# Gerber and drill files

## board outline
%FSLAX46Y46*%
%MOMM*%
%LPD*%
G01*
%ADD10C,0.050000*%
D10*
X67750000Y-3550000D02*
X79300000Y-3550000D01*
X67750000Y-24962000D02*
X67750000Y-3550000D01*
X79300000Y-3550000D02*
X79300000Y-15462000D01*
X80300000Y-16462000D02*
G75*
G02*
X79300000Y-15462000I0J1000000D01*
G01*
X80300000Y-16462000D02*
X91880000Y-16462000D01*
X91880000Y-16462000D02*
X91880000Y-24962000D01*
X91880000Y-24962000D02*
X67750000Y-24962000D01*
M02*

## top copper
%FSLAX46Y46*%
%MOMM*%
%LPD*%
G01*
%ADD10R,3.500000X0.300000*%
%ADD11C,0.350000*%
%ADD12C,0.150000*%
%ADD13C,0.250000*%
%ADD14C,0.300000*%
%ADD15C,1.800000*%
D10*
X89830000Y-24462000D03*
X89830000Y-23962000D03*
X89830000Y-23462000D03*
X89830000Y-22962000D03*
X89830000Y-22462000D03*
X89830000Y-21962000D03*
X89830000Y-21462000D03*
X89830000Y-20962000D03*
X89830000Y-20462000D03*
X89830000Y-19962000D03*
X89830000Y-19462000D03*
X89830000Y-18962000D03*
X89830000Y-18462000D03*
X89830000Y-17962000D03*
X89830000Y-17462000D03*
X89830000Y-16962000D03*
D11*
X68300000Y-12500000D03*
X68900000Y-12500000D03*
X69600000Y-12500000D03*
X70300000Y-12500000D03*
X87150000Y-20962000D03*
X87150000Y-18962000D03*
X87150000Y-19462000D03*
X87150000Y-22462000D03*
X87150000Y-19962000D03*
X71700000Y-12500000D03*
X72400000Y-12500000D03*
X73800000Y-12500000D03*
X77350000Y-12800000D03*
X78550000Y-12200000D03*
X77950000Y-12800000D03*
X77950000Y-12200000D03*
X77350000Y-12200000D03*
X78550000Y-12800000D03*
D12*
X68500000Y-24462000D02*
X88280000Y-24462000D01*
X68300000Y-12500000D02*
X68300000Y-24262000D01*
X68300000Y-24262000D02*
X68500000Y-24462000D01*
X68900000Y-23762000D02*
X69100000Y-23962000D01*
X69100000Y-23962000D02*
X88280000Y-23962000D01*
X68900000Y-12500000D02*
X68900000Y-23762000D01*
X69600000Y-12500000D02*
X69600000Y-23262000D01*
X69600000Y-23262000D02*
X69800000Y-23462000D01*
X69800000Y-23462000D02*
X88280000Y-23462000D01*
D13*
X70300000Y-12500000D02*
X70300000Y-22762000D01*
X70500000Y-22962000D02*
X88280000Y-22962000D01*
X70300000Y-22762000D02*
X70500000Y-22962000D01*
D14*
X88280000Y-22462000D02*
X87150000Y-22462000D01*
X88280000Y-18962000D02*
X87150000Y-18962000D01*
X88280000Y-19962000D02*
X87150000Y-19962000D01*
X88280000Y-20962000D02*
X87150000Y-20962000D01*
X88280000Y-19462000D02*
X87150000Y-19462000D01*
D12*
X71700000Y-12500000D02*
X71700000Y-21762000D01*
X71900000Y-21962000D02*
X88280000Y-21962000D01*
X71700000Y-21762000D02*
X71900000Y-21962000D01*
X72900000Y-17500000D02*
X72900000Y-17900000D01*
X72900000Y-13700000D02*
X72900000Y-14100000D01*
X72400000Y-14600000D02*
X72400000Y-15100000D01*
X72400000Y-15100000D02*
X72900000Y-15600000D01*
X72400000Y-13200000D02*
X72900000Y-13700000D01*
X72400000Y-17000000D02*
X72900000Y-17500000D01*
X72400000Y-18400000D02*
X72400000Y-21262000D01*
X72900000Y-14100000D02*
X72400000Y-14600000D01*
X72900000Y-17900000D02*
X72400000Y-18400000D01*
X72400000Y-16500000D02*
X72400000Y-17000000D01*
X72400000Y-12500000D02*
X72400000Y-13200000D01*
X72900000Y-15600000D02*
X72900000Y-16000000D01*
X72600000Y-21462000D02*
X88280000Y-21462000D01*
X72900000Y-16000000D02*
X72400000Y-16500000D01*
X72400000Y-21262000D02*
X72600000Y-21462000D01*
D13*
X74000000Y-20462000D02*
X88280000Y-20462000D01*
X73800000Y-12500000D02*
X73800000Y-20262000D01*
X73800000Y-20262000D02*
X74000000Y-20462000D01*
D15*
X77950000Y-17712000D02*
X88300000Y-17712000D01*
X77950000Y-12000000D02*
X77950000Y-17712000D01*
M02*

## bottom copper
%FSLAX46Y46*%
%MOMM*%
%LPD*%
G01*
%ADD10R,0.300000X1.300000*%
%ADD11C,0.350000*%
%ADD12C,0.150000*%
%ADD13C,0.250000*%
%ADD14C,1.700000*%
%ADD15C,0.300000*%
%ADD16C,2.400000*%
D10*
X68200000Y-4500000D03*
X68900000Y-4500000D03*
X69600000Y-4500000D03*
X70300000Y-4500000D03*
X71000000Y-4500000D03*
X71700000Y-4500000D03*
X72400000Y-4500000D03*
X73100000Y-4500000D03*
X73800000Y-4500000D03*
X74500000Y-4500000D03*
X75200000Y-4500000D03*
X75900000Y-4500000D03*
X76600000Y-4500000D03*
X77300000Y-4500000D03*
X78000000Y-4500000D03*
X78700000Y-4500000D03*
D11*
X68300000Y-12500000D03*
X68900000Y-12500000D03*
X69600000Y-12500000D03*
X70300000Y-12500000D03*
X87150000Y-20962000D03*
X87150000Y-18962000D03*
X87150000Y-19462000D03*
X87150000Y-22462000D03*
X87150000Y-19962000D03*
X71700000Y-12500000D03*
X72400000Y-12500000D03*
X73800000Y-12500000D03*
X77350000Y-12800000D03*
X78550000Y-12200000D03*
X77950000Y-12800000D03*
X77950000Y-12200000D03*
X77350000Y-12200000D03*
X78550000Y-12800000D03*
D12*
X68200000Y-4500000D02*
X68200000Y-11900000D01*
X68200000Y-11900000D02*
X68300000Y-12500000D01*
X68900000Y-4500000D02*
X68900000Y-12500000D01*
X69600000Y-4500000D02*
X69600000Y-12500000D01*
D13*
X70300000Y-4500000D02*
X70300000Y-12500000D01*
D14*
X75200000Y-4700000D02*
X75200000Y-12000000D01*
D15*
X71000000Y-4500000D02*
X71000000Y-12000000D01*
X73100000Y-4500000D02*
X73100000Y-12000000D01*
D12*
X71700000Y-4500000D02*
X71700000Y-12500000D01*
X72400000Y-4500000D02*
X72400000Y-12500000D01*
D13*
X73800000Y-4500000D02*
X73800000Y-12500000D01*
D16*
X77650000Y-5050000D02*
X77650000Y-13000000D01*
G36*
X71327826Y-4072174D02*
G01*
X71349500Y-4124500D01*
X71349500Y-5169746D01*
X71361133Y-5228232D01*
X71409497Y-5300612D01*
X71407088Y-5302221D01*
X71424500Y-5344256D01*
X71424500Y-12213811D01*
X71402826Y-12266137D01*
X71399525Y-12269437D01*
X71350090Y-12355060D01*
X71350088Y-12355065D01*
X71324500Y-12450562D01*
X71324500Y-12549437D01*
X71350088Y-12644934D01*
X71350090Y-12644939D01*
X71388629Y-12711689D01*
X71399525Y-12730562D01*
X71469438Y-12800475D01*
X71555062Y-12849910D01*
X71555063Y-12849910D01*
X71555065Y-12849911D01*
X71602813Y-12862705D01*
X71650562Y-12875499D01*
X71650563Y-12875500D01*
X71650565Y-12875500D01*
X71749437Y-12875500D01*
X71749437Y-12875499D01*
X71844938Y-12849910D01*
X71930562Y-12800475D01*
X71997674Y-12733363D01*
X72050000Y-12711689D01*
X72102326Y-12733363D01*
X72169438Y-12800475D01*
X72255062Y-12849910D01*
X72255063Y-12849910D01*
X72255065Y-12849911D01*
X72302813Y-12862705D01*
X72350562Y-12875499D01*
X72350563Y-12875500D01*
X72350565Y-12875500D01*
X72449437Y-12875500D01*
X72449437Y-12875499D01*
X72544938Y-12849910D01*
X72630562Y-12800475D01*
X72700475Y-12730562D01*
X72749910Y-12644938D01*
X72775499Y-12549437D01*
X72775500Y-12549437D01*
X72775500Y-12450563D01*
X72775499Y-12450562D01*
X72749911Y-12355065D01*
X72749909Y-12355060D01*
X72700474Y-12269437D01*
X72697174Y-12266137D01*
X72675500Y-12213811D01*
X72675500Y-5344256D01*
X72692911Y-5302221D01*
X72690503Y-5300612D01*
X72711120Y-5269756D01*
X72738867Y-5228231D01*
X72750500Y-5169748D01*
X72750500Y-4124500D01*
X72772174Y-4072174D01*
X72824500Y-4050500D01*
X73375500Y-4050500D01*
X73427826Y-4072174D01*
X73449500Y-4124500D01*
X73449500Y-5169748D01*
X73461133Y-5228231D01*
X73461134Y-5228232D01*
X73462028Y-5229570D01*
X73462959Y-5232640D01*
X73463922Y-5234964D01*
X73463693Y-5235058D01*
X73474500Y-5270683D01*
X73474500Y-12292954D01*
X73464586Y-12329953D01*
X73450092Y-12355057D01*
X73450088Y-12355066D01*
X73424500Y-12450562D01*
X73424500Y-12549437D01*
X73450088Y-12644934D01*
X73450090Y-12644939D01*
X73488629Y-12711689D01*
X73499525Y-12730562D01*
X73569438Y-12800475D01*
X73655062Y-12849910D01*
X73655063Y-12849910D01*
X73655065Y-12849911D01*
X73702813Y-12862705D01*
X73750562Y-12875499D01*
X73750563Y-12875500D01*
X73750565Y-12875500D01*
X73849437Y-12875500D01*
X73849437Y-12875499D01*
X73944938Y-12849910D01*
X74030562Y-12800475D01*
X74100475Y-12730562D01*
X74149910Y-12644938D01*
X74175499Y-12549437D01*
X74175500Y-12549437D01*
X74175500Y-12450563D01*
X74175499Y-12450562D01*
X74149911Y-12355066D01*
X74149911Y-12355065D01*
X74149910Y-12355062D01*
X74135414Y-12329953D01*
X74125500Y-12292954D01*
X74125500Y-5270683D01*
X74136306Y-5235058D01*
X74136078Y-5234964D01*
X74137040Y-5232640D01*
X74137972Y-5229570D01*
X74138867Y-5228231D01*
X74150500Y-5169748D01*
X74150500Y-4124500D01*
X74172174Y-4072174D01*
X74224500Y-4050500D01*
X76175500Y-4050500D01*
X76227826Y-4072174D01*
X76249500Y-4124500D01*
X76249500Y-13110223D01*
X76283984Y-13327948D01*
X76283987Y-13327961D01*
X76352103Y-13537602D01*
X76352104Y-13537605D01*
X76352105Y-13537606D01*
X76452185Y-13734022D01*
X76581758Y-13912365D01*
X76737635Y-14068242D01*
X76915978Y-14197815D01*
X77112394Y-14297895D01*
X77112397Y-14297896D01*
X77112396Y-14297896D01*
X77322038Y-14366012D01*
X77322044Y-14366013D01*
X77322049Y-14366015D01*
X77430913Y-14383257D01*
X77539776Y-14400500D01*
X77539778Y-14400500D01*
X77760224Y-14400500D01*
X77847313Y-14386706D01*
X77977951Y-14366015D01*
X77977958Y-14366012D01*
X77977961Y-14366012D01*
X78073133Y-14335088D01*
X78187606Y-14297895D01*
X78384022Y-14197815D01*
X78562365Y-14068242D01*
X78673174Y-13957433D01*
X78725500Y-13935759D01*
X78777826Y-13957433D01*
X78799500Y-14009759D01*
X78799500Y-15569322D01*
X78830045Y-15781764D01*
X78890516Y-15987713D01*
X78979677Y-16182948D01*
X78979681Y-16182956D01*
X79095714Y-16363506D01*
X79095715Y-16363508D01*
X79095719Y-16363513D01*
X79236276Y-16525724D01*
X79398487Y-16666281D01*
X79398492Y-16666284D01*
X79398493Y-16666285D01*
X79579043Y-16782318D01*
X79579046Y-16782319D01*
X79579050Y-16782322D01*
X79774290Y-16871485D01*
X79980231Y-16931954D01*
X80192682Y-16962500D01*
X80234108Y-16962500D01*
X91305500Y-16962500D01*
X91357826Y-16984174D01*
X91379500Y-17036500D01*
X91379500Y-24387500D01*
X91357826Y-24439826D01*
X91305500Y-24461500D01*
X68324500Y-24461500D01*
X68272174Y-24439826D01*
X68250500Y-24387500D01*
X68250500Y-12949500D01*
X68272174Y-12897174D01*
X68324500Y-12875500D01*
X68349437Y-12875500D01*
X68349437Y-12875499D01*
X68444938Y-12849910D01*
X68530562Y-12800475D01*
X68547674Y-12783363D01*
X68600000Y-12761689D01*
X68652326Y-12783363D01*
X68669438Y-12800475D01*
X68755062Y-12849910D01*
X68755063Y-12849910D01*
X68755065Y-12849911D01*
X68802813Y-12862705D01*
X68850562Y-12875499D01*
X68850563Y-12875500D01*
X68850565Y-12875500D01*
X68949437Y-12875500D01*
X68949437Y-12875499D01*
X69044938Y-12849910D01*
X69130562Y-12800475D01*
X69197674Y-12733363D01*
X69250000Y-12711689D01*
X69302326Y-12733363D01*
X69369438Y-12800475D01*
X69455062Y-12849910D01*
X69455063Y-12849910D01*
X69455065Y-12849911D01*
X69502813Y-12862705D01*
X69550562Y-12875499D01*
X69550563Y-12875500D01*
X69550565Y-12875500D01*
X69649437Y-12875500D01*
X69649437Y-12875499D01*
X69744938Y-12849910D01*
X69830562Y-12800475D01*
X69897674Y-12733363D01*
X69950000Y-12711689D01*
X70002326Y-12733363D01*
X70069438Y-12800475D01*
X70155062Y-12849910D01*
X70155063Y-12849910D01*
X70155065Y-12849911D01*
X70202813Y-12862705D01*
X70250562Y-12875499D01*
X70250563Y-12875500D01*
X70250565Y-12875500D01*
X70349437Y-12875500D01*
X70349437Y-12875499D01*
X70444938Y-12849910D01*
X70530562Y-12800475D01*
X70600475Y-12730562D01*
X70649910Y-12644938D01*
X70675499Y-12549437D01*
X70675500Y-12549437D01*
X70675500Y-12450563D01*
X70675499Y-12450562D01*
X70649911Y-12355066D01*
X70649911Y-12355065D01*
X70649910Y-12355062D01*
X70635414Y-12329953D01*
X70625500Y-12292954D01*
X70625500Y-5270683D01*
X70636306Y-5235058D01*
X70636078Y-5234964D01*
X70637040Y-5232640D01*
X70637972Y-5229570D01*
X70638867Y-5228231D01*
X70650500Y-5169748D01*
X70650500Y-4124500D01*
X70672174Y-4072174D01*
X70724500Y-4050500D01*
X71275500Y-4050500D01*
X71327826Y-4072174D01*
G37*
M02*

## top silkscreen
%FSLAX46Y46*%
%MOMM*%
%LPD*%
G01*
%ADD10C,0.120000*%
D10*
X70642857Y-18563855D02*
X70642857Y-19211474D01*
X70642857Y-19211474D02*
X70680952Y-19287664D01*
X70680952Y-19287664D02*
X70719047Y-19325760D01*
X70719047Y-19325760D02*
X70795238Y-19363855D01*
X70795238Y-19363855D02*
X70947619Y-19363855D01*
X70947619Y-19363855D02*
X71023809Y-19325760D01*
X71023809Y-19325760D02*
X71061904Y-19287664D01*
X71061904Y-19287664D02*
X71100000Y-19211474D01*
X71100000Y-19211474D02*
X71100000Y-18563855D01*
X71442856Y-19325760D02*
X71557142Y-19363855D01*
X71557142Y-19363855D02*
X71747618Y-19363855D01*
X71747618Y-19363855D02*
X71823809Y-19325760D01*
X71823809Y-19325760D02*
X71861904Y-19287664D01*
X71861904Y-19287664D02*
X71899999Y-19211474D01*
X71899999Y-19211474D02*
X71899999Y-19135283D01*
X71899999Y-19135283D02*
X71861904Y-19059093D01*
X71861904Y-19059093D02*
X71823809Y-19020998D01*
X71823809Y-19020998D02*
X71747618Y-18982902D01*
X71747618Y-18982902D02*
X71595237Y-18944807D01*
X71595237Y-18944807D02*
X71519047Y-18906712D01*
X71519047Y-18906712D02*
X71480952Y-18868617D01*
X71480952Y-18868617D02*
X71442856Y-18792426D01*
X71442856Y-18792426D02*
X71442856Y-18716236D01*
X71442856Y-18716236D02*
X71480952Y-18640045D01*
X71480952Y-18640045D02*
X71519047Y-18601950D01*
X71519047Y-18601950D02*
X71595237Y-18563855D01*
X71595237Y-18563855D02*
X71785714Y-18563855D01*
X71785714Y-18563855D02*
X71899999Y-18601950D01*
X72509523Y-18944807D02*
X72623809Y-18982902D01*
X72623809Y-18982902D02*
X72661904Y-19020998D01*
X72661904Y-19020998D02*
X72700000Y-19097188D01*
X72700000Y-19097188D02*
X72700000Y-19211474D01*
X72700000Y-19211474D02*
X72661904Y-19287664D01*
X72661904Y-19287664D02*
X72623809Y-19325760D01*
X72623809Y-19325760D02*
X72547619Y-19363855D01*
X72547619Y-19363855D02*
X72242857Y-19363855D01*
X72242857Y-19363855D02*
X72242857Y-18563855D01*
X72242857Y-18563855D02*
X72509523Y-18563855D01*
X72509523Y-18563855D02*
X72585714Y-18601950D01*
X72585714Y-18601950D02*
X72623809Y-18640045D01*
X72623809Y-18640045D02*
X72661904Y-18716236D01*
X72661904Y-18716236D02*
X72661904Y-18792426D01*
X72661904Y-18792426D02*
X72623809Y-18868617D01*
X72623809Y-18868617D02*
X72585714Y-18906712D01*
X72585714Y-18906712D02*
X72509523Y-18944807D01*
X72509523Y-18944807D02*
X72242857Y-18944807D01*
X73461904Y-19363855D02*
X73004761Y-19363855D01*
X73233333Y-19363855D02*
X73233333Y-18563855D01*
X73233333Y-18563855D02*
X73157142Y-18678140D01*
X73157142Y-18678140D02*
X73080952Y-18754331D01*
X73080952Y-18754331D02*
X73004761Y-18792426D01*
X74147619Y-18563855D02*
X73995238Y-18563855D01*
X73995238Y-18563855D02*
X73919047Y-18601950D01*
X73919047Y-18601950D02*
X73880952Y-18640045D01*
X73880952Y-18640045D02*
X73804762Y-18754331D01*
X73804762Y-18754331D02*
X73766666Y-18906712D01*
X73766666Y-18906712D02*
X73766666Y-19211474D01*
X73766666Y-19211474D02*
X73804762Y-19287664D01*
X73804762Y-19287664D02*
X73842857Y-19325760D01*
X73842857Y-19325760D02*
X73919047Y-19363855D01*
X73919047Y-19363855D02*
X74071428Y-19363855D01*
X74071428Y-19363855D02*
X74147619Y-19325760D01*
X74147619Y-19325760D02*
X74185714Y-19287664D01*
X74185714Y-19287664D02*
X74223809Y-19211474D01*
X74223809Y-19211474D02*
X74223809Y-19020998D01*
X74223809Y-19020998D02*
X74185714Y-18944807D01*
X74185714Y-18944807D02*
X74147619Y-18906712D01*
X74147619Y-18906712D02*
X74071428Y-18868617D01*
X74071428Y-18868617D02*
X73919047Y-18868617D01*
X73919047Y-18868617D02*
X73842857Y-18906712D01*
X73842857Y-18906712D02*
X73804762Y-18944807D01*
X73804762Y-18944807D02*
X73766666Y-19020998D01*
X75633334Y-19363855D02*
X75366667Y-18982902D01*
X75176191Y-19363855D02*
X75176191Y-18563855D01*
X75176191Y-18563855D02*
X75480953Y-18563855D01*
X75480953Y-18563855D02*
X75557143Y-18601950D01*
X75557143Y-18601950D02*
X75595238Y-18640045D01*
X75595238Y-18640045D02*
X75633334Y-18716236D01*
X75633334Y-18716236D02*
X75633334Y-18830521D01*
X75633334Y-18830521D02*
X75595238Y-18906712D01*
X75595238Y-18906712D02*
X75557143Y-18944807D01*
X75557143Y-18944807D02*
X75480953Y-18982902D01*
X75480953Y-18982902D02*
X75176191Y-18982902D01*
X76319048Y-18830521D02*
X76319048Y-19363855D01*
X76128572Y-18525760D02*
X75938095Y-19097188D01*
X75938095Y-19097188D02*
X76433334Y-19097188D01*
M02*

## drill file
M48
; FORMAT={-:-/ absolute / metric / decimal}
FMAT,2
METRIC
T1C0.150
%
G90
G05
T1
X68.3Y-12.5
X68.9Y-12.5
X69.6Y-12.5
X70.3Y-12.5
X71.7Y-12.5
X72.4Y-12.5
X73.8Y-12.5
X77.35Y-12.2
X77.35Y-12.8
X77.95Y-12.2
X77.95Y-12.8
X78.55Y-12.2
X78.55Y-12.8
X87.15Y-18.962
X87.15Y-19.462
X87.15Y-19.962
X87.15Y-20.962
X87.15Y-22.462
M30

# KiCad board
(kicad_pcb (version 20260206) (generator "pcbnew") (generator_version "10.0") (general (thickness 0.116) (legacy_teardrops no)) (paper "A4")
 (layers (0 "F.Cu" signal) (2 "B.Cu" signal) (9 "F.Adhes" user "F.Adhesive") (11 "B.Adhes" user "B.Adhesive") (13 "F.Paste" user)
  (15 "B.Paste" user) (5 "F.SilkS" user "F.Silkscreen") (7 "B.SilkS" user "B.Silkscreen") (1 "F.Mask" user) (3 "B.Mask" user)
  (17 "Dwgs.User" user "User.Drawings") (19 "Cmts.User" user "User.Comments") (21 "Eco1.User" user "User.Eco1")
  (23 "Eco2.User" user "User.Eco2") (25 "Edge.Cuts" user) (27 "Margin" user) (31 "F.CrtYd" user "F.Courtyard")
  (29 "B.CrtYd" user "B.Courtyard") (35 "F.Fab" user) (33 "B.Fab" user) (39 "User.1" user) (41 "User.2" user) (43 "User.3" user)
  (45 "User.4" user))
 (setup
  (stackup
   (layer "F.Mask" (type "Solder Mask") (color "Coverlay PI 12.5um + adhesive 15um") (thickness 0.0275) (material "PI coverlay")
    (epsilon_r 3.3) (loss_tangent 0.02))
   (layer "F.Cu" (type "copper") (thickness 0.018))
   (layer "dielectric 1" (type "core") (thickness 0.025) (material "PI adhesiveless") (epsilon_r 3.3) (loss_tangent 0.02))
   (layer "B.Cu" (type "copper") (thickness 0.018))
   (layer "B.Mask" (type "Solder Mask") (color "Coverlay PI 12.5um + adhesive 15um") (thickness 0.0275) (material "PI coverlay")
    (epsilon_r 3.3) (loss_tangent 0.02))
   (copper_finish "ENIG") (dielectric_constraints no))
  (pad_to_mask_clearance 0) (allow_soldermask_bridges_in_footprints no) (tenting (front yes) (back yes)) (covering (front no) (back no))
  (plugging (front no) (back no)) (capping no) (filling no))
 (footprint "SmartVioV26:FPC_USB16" (layer "F.Cu") (at 0 0)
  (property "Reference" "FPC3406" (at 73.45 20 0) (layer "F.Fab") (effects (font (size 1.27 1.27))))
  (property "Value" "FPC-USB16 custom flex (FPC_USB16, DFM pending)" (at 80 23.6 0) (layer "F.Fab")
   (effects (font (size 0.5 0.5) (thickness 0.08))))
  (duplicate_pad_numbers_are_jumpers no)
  (pad "S1" smd rect (at 68.2 4.5) (size 0.3 1.3) (layers "B.Cu" "B.Mask") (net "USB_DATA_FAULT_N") (solder_mask_margin 0.05)
   (thermal_bridge_angle 45))
  (pad "S2" smd rect (at 68.9 4.5) (size 0.3 1.3) (layers "B.Cu" "B.Mask") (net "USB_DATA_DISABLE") (solder_mask_margin 0.05)
   (thermal_bridge_angle 45))
  (pad "S3" smd rect (at 69.6 4.5) (size 0.3 1.3) (layers "B.Cu" "B.Mask") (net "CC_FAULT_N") (solder_mask_margin 0.05)
   (thermal_bridge_angle 45))
  (pad "S4" smd rect (at 70.3 4.5) (size 0.3 1.3) (layers "B.Cu" "B.Mask") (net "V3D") (solder_mask_margin 0.05) (thermal_bridge_angle 45))
  (pad "S5" smd rect (at 71 4.5) (size 0.3 1.3) (layers "B.Cu" "B.Mask") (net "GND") (solder_mask_margin 0.05) (thermal_bridge_angle 45))
  (pad "S6" smd rect (at 71.7 4.5) (size 0.3 1.3) (layers "B.Cu" "B.Mask") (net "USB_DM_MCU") (solder_mask_margin 0.05)
   (thermal_bridge_angle 45))
  (pad "S7" smd rect (at 72.4 4.5) (size 0.3 1.3) (layers "B.Cu" "B.Mask") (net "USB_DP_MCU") (solder_mask_margin 0.05)
   (thermal_bridge_angle 45))
  (pad "S8" smd rect (at 73.1 4.5) (size 0.3 1.3) (layers "B.Cu" "B.Mask") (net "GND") (solder_mask_margin 0.05) (thermal_bridge_angle 45))
  (pad "S9" smd rect (at 73.8 4.5) (size 0.3 1.3) (layers "B.Cu" "B.Mask") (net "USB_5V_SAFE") (solder_mask_margin 0.05)
   (thermal_bridge_angle 45))
  (pad "S10" smd rect (at 74.5 4.5) (size 0.3 1.3) (layers "B.Cu" "B.Mask") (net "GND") (solder_mask_margin 0.05) (thermal_bridge_angle 45))
  (pad "S11" smd rect (at 75.2 4.5) (size 0.3 1.3) (layers "B.Cu" "B.Mask") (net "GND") (solder_mask_margin 0.05) (thermal_bridge_angle 45))
  (pad "S12" smd rect (at 75.9 4.5) (size 0.3 1.3) (layers "B.Cu" "B.Mask") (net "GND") (solder_mask_margin 0.05) (thermal_bridge_angle 45))
  (pad "S13" smd rect (at 76.6 4.5) (size 0.3 1.3) (layers "B.Cu" "B.Mask") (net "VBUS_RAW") (solder_mask_margin 0.05)
   (thermal_bridge_angle 45))
  (pad "S14" smd rect (at 77.3 4.5) (size 0.3 1.3) (layers "B.Cu" "B.Mask") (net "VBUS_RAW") (solder_mask_margin 0.05)
   (thermal_bridge_angle 45))
  (pad "S15" smd rect (at 78 4.5) (size 0.3 1.3) (layers "B.Cu" "B.Mask") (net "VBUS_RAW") (solder_mask_margin 0.05)
   (thermal_bridge_angle 45))
  (pad "S16" smd rect (at 78.7 4.5) (size 0.3 1.3) (layers "B.Cu" "B.Mask") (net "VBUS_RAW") (solder_mask_margin 0.05)
   (thermal_bridge_angle 45))
  (pad "T1" smd rect (at 89.83 24.462) (size 3.5 0.3) (layers "F.Cu" "F.Mask") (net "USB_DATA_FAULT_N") (solder_mask_margin 0)
   (thermal_bridge_angle 45))
  (pad "T2" smd rect (at 89.83 23.962) (size 3.5 0.3) (layers "F.Cu" "F.Mask") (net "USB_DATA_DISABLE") (solder_mask_margin 0)
   (thermal_bridge_angle 45))
  (pad "T3" smd rect (at 89.83 23.462) (size 3.5 0.3) (layers "F.Cu" "F.Mask") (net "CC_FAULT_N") (solder_mask_margin 0)
   (thermal_bridge_angle 45))
  (pad "T4" smd rect (at 89.83 22.962) (size 3.5 0.3) (layers "F.Cu" "F.Mask") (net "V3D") (solder_mask_margin 0) (thermal_bridge_angle 45))
  (pad "T5" smd rect (at 89.83 22.462) (size 3.5 0.3) (layers "F.Cu" "F.Mask") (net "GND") (solder_mask_margin 0) (thermal_bridge_angle 45))
  (pad "T6" smd rect (at 89.83 21.962) (size 3.5 0.3) (layers "F.Cu" "F.Mask") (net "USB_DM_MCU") (solder_mask_margin 0)
   (thermal_bridge_angle 45))
  (pad "T7" smd rect (at 89.83 21.462) (size 3.5 0.3) (layers "F.Cu" "F.Mask") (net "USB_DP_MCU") (solder_mask_margin 0)
   (thermal_bridge_angle 45))
  (pad "T8" smd rect (at 89.83 20.962) (size 3.5 0.3) (layers "F.Cu" "F.Mask") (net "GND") (solder_mask_margin 0) (thermal_bridge_angle 45))
  (pad "T9" smd rect (at 89.83 20.462) (size 3.5 0.3) (layers "F.Cu" "F.Mask") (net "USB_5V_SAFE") (solder_mask_margin 0)
   (thermal_bridge_angle 45))
  (pad "T10" smd rect (at 89.83 19.962) (size 3.5 0.3) (layers "F.Cu" "F.Mask") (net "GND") (solder_mask_margin 0) (thermal_bridge_angle 45))
  (pad "T11" smd rect (at 89.83 19.462) (size 3.5 0.3) (layers "F.Cu" "F.Mask") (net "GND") (solder_mask_margin 0) (thermal_bridge_angle 45))
  (pad "T12" smd rect (at 89.83 18.962) (size 3.5 0.3) (layers "F.Cu" "F.Mask") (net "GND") (solder_mask_margin 0) (thermal_bridge_angle 45))
  (pad "T13" smd rect (at 89.83 18.462) (size 3.5 0.3) (layers "F.Cu" "F.Mask") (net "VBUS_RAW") (solder_mask_margin 0)
   (thermal_bridge_angle 45))
  (pad "T14" smd rect (at 89.83 17.962) (size 3.5 0.3) (layers "F.Cu" "F.Mask") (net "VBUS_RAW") (solder_mask_margin 0)
   (thermal_bridge_angle 45))
  (pad "T15" smd rect (at 89.83 17.462) (size 3.5 0.3) (layers "F.Cu" "F.Mask") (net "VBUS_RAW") (solder_mask_margin 0)
   (thermal_bridge_angle 45))
  (pad "T16" smd rect (at 89.83 16.962) (size 3.5 0.3) (layers "F.Cu" "F.Mask") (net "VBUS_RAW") (solder_mask_margin 0)
   (thermal_bridge_angle 45)))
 (gr_line (start 67.75 3.55) (end 79.3 3.55) (stroke (width 0.05) (type default)) (layer "Edge.Cuts"))
 (gr_line (start 67.75 24.962) (end 67.75 3.55) (stroke (width 0.05) (type default)) (layer "Edge.Cuts"))
 (gr_line (start 79.3 3.55) (end 79.3 15.462) (stroke (width 0.05) (type default)) (layer "Edge.Cuts"))
 (gr_arc (start 80.3 16.462) (mid 79.592893 16.169107) (end 79.3 15.462) (stroke (width 0.05) (type default)) (layer "Edge.Cuts"))
 (gr_line (start 80.3 16.462) (end 91.88 16.462) (stroke (width 0.05) (type default)) (layer "Edge.Cuts"))
 (gr_line (start 91.88 16.462) (end 91.88 24.962) (stroke (width 0.05) (type default)) (layer "Edge.Cuts"))
 (gr_line (start 91.88 24.962) (end 67.75 24.962) (stroke (width 0.05) (type default)) (layer "Edge.Cuts"))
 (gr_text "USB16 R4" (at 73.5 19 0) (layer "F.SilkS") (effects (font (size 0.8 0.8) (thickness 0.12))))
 (segment (start 68.5 24.462) (end 88.28 24.462) (width 0.15) (layer "F.Cu") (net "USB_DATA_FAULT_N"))
 (segment (start 68.3 12.5) (end 68.3 24.262) (width 0.15) (layer "F.Cu") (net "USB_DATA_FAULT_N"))
 (segment (start 68.3 24.262) (end 68.5 24.462) (width 0.15) (layer "F.Cu") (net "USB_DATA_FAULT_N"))
 (via (at 68.3 12.5) (size 0.35) (drill 0.15) (layers "F.Cu" "B.Cu") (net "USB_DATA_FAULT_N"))
 (segment (start 68.2 4.5) (end 68.2 11.9) (width 0.15) (layer "B.Cu") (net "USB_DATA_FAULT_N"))
 (segment (start 68.2 11.9) (end 68.3 12.5) (width 0.15) (layer "B.Cu") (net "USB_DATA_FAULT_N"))
 (segment (start 68.9 23.762) (end 69.1 23.962) (width 0.15) (layer "F.Cu") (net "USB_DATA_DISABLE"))
 (segment (start 69.1 23.962) (end 88.28 23.962) (width 0.15) (layer "F.Cu") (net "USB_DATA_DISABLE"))
 (segment (start 68.9 12.5) (end 68.9 23.762) (width 0.15) (layer "F.Cu") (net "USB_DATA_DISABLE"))
 (via (at 68.9 12.5) (size 0.35) (drill 0.15) (layers "F.Cu" "B.Cu") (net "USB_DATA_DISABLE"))
 (segment (start 68.9 4.5) (end 68.9 12.5) (width 0.15) (layer "B.Cu") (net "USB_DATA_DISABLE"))
 (segment (start 69.6 12.5) (end 69.6 23.262) (width 0.15) (layer "F.Cu") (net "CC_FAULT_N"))
 (segment (start 69.6 23.262) (end 69.8 23.462) (width 0.15) (layer "F.Cu") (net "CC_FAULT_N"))
 (segment (start 69.8 23.462) (end 88.28 23.462) (width 0.15) (layer "F.Cu") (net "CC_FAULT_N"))
 (via (at 69.6 12.5) (size 0.35) (drill 0.15) (layers "F.Cu" "B.Cu") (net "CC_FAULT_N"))
 (segment (start 69.6 4.5) (end 69.6 12.5) (width 0.15) (layer "B.Cu") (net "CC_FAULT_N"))
 (segment (start 70.3 12.5) (end 70.3 22.762) (width 0.25) (layer "F.Cu") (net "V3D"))
 (segment (start 70.5 22.962) (end 88.28 22.962) (width 0.25) (layer "F.Cu") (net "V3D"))
 (segment (start 70.3 22.762) (end 70.5 22.962) (width 0.25) (layer "F.Cu") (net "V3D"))
 (via (at 70.3 12.5) (size 0.35) (drill 0.15) (layers "F.Cu" "B.Cu") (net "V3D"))
 (segment (start 70.3 4.5) (end 70.3 12.5) (width 0.25) (layer "B.Cu") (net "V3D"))
 (segment (start 88.28 22.462) (end 87.15 22.462) (width 0.3) (layer "F.Cu") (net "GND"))
 (segment (start 88.28 18.962) (end 87.15 18.962) (width 0.3) (layer "F.Cu") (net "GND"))
 (segment (start 88.28 19.962) (end 87.15 19.962) (width 0.3) (layer "F.Cu") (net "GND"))
 (segment (start 88.28 20.962) (end 87.15 20.962) (width 0.3) (layer "F.Cu") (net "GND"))
 (segment (start 88.28 19.462) (end 87.15 19.462) (width 0.3) (layer "F.Cu") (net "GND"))
 (via (at 87.15 20.962) (size 0.35) (drill 0.15) (layers "F.Cu" "B.Cu") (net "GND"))
 (via (at 87.15 18.962) (size 0.35) (drill 0.15) (layers "F.Cu" "B.Cu") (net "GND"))
 (via (at 87.15 19.462) (size 0.35) (drill 0.15) (layers "F.Cu" "B.Cu") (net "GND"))
 (via (at 87.15 22.462) (size 0.35) (drill 0.15) (layers "F.Cu" "B.Cu") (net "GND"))
 (via (at 87.15 19.962) (size 0.35) (drill 0.15) (layers "F.Cu" "B.Cu") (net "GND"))
 (segment (start 75.2 4.7) (end 75.2 12) (width 1.7) (layer "B.Cu") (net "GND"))
 (segment (start 71 4.5) (end 71 12) (width 0.3) (layer "B.Cu") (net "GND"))
 (segment (start 73.1 4.5) (end 73.1 12) (width 0.3) (layer "B.Cu") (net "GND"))
 (segment (start 71.7 12.5) (end 71.7 21.762) (width 0.15) (layer "F.Cu") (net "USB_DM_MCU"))
 (segment (start 71.9 21.962) (end 88.28 21.962) (width 0.15) (layer "F.Cu") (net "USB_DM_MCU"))
 (segment (start 71.7 21.762) (end 71.9 21.962) (width 0.15) (layer "F.Cu") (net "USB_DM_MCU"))
 (via (at 71.7 12.5) (size 0.35) (drill 0.15) (layers "F.Cu" "B.Cu") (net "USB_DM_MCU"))
 (segment (start 71.7 4.5) (end 71.7 12.5) (width 0.15) (layer "B.Cu") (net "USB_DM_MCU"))
 (segment (start 72.9 17.5) (end 72.9 17.9) (width 0.15) (layer "F.Cu") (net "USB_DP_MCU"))
 (segment (start 72.9 13.7) (end 72.9 14.1) (width 0.15) (layer "F.Cu") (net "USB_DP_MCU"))
 (segment (start 72.4 14.6) (end 72.4 15.1) (width 0.15) (layer "F.Cu") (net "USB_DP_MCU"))
 (segment (start 72.4 15.1) (end 72.9 15.6) (width 0.15) (layer "F.Cu") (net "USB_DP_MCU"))
 (segment (start 72.4 13.2) (end 72.9 13.7) (width 0.15) (layer "F.Cu") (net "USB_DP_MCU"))
 (segment (start 72.4 17) (end 72.9 17.5) (width 0.15) (layer "F.Cu") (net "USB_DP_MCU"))
 (segment (start 72.4 18.4) (end 72.4 21.262) (width 0.15) (layer "F.Cu") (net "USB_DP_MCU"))
 (segment (start 72.9 14.1) (end 72.4 14.6) (width 0.15) (layer "F.Cu") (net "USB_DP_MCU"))
 (segment (start 72.9 17.9) (end 72.4 18.4) (width 0.15) (layer "F.Cu") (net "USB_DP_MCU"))
 (segment (start 72.4 16.5) (end 72.4 17) (width 0.15) (layer "F.Cu") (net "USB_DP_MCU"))
 (segment (start 72.4 12.5) (end 72.4 13.2) (width 0.15) (layer "F.Cu") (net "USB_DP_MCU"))
 (segment (start 72.9 15.6) (end 72.9 16) (width 0.15) (layer "F.Cu") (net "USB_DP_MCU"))
 (segment (start 72.6 21.462) (end 88.28 21.462) (width 0.15) (layer "F.Cu") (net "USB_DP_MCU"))
 (segment (start 72.9 16) (end 72.4 16.5) (width 0.15) (layer "F.Cu") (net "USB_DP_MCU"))
 (segment (start 72.4 21.262) (end 72.6 21.462) (width 0.15) (layer "F.Cu") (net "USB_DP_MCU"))
 (via (at 72.4 12.5) (size 0.35) (drill 0.15) (layers "F.Cu" "B.Cu") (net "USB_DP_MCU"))
 (segment (start 72.4 4.5) (end 72.4 12.5) (width 0.15) (layer "B.Cu") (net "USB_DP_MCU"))
 (segment (start 74 20.462) (end 88.28 20.462) (width 0.25) (layer "F.Cu") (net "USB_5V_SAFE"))
 (segment (start 73.8 12.5) (end 73.8 20.262) (width 0.25) (layer "F.Cu") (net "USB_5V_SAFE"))
 (segment (start 73.8 20.262) (end 74 20.462) (width 0.25) (layer "F.Cu") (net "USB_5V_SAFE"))
 (via (at 73.8 12.5) (size 0.35) (drill 0.15) (layers "F.Cu" "B.Cu") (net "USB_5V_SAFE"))
 (segment (start 73.8 4.5) (end 73.8 12.5) (width 0.25) (layer "B.Cu") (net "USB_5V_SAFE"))
 (segment (start 77.95 17.712) (end 88.3 17.712) (width 1.8) (layer "F.Cu") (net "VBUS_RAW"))
 (segment (start 77.95 12) (end 77.95 17.712) (width 1.8) (layer "F.Cu") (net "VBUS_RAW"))
 (via (at 77.35 12.8) (size 0.35) (drill 0.15) (layers "F.Cu" "B.Cu") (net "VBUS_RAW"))
 (via (at 78.55 12.2) (size 0.35) (drill 0.15) (layers "F.Cu" "B.Cu") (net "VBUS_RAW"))
 (via (at 77.95 12.8) (size 0.35) (drill 0.15) (layers "F.Cu" "B.Cu") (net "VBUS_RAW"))
 (via (at 77.95 12.2) (size 0.35) (drill 0.15) (layers "F.Cu" "B.Cu") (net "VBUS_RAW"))
 (via (at 77.35 12.2) (size 0.35) (drill 0.15) (layers "F.Cu" "B.Cu") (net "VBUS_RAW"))
 (via (at 78.55 12.8) (size 0.35) (drill 0.15) (layers "F.Cu" "B.Cu") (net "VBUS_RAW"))
 (segment (start 77.65 5.05) (end 77.65 13) (width 2.4) (layer "B.Cu") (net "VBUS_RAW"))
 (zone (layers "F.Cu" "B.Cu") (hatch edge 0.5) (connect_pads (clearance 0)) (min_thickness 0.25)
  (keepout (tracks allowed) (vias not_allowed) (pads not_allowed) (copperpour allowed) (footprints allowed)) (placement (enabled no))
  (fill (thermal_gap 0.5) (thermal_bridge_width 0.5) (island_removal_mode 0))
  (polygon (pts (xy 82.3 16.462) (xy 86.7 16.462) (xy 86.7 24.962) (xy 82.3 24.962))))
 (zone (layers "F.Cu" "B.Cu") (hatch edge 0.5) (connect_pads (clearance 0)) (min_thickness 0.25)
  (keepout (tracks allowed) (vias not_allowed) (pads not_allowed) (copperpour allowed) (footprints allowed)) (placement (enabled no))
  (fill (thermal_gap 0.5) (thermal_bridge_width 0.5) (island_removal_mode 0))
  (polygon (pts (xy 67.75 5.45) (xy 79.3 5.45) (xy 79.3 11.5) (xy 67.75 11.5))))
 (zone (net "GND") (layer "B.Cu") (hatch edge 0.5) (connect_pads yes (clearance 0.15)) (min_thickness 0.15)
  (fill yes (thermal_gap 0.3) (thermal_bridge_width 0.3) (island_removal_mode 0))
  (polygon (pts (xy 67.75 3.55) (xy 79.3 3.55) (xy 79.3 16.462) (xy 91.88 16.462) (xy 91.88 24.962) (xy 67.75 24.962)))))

